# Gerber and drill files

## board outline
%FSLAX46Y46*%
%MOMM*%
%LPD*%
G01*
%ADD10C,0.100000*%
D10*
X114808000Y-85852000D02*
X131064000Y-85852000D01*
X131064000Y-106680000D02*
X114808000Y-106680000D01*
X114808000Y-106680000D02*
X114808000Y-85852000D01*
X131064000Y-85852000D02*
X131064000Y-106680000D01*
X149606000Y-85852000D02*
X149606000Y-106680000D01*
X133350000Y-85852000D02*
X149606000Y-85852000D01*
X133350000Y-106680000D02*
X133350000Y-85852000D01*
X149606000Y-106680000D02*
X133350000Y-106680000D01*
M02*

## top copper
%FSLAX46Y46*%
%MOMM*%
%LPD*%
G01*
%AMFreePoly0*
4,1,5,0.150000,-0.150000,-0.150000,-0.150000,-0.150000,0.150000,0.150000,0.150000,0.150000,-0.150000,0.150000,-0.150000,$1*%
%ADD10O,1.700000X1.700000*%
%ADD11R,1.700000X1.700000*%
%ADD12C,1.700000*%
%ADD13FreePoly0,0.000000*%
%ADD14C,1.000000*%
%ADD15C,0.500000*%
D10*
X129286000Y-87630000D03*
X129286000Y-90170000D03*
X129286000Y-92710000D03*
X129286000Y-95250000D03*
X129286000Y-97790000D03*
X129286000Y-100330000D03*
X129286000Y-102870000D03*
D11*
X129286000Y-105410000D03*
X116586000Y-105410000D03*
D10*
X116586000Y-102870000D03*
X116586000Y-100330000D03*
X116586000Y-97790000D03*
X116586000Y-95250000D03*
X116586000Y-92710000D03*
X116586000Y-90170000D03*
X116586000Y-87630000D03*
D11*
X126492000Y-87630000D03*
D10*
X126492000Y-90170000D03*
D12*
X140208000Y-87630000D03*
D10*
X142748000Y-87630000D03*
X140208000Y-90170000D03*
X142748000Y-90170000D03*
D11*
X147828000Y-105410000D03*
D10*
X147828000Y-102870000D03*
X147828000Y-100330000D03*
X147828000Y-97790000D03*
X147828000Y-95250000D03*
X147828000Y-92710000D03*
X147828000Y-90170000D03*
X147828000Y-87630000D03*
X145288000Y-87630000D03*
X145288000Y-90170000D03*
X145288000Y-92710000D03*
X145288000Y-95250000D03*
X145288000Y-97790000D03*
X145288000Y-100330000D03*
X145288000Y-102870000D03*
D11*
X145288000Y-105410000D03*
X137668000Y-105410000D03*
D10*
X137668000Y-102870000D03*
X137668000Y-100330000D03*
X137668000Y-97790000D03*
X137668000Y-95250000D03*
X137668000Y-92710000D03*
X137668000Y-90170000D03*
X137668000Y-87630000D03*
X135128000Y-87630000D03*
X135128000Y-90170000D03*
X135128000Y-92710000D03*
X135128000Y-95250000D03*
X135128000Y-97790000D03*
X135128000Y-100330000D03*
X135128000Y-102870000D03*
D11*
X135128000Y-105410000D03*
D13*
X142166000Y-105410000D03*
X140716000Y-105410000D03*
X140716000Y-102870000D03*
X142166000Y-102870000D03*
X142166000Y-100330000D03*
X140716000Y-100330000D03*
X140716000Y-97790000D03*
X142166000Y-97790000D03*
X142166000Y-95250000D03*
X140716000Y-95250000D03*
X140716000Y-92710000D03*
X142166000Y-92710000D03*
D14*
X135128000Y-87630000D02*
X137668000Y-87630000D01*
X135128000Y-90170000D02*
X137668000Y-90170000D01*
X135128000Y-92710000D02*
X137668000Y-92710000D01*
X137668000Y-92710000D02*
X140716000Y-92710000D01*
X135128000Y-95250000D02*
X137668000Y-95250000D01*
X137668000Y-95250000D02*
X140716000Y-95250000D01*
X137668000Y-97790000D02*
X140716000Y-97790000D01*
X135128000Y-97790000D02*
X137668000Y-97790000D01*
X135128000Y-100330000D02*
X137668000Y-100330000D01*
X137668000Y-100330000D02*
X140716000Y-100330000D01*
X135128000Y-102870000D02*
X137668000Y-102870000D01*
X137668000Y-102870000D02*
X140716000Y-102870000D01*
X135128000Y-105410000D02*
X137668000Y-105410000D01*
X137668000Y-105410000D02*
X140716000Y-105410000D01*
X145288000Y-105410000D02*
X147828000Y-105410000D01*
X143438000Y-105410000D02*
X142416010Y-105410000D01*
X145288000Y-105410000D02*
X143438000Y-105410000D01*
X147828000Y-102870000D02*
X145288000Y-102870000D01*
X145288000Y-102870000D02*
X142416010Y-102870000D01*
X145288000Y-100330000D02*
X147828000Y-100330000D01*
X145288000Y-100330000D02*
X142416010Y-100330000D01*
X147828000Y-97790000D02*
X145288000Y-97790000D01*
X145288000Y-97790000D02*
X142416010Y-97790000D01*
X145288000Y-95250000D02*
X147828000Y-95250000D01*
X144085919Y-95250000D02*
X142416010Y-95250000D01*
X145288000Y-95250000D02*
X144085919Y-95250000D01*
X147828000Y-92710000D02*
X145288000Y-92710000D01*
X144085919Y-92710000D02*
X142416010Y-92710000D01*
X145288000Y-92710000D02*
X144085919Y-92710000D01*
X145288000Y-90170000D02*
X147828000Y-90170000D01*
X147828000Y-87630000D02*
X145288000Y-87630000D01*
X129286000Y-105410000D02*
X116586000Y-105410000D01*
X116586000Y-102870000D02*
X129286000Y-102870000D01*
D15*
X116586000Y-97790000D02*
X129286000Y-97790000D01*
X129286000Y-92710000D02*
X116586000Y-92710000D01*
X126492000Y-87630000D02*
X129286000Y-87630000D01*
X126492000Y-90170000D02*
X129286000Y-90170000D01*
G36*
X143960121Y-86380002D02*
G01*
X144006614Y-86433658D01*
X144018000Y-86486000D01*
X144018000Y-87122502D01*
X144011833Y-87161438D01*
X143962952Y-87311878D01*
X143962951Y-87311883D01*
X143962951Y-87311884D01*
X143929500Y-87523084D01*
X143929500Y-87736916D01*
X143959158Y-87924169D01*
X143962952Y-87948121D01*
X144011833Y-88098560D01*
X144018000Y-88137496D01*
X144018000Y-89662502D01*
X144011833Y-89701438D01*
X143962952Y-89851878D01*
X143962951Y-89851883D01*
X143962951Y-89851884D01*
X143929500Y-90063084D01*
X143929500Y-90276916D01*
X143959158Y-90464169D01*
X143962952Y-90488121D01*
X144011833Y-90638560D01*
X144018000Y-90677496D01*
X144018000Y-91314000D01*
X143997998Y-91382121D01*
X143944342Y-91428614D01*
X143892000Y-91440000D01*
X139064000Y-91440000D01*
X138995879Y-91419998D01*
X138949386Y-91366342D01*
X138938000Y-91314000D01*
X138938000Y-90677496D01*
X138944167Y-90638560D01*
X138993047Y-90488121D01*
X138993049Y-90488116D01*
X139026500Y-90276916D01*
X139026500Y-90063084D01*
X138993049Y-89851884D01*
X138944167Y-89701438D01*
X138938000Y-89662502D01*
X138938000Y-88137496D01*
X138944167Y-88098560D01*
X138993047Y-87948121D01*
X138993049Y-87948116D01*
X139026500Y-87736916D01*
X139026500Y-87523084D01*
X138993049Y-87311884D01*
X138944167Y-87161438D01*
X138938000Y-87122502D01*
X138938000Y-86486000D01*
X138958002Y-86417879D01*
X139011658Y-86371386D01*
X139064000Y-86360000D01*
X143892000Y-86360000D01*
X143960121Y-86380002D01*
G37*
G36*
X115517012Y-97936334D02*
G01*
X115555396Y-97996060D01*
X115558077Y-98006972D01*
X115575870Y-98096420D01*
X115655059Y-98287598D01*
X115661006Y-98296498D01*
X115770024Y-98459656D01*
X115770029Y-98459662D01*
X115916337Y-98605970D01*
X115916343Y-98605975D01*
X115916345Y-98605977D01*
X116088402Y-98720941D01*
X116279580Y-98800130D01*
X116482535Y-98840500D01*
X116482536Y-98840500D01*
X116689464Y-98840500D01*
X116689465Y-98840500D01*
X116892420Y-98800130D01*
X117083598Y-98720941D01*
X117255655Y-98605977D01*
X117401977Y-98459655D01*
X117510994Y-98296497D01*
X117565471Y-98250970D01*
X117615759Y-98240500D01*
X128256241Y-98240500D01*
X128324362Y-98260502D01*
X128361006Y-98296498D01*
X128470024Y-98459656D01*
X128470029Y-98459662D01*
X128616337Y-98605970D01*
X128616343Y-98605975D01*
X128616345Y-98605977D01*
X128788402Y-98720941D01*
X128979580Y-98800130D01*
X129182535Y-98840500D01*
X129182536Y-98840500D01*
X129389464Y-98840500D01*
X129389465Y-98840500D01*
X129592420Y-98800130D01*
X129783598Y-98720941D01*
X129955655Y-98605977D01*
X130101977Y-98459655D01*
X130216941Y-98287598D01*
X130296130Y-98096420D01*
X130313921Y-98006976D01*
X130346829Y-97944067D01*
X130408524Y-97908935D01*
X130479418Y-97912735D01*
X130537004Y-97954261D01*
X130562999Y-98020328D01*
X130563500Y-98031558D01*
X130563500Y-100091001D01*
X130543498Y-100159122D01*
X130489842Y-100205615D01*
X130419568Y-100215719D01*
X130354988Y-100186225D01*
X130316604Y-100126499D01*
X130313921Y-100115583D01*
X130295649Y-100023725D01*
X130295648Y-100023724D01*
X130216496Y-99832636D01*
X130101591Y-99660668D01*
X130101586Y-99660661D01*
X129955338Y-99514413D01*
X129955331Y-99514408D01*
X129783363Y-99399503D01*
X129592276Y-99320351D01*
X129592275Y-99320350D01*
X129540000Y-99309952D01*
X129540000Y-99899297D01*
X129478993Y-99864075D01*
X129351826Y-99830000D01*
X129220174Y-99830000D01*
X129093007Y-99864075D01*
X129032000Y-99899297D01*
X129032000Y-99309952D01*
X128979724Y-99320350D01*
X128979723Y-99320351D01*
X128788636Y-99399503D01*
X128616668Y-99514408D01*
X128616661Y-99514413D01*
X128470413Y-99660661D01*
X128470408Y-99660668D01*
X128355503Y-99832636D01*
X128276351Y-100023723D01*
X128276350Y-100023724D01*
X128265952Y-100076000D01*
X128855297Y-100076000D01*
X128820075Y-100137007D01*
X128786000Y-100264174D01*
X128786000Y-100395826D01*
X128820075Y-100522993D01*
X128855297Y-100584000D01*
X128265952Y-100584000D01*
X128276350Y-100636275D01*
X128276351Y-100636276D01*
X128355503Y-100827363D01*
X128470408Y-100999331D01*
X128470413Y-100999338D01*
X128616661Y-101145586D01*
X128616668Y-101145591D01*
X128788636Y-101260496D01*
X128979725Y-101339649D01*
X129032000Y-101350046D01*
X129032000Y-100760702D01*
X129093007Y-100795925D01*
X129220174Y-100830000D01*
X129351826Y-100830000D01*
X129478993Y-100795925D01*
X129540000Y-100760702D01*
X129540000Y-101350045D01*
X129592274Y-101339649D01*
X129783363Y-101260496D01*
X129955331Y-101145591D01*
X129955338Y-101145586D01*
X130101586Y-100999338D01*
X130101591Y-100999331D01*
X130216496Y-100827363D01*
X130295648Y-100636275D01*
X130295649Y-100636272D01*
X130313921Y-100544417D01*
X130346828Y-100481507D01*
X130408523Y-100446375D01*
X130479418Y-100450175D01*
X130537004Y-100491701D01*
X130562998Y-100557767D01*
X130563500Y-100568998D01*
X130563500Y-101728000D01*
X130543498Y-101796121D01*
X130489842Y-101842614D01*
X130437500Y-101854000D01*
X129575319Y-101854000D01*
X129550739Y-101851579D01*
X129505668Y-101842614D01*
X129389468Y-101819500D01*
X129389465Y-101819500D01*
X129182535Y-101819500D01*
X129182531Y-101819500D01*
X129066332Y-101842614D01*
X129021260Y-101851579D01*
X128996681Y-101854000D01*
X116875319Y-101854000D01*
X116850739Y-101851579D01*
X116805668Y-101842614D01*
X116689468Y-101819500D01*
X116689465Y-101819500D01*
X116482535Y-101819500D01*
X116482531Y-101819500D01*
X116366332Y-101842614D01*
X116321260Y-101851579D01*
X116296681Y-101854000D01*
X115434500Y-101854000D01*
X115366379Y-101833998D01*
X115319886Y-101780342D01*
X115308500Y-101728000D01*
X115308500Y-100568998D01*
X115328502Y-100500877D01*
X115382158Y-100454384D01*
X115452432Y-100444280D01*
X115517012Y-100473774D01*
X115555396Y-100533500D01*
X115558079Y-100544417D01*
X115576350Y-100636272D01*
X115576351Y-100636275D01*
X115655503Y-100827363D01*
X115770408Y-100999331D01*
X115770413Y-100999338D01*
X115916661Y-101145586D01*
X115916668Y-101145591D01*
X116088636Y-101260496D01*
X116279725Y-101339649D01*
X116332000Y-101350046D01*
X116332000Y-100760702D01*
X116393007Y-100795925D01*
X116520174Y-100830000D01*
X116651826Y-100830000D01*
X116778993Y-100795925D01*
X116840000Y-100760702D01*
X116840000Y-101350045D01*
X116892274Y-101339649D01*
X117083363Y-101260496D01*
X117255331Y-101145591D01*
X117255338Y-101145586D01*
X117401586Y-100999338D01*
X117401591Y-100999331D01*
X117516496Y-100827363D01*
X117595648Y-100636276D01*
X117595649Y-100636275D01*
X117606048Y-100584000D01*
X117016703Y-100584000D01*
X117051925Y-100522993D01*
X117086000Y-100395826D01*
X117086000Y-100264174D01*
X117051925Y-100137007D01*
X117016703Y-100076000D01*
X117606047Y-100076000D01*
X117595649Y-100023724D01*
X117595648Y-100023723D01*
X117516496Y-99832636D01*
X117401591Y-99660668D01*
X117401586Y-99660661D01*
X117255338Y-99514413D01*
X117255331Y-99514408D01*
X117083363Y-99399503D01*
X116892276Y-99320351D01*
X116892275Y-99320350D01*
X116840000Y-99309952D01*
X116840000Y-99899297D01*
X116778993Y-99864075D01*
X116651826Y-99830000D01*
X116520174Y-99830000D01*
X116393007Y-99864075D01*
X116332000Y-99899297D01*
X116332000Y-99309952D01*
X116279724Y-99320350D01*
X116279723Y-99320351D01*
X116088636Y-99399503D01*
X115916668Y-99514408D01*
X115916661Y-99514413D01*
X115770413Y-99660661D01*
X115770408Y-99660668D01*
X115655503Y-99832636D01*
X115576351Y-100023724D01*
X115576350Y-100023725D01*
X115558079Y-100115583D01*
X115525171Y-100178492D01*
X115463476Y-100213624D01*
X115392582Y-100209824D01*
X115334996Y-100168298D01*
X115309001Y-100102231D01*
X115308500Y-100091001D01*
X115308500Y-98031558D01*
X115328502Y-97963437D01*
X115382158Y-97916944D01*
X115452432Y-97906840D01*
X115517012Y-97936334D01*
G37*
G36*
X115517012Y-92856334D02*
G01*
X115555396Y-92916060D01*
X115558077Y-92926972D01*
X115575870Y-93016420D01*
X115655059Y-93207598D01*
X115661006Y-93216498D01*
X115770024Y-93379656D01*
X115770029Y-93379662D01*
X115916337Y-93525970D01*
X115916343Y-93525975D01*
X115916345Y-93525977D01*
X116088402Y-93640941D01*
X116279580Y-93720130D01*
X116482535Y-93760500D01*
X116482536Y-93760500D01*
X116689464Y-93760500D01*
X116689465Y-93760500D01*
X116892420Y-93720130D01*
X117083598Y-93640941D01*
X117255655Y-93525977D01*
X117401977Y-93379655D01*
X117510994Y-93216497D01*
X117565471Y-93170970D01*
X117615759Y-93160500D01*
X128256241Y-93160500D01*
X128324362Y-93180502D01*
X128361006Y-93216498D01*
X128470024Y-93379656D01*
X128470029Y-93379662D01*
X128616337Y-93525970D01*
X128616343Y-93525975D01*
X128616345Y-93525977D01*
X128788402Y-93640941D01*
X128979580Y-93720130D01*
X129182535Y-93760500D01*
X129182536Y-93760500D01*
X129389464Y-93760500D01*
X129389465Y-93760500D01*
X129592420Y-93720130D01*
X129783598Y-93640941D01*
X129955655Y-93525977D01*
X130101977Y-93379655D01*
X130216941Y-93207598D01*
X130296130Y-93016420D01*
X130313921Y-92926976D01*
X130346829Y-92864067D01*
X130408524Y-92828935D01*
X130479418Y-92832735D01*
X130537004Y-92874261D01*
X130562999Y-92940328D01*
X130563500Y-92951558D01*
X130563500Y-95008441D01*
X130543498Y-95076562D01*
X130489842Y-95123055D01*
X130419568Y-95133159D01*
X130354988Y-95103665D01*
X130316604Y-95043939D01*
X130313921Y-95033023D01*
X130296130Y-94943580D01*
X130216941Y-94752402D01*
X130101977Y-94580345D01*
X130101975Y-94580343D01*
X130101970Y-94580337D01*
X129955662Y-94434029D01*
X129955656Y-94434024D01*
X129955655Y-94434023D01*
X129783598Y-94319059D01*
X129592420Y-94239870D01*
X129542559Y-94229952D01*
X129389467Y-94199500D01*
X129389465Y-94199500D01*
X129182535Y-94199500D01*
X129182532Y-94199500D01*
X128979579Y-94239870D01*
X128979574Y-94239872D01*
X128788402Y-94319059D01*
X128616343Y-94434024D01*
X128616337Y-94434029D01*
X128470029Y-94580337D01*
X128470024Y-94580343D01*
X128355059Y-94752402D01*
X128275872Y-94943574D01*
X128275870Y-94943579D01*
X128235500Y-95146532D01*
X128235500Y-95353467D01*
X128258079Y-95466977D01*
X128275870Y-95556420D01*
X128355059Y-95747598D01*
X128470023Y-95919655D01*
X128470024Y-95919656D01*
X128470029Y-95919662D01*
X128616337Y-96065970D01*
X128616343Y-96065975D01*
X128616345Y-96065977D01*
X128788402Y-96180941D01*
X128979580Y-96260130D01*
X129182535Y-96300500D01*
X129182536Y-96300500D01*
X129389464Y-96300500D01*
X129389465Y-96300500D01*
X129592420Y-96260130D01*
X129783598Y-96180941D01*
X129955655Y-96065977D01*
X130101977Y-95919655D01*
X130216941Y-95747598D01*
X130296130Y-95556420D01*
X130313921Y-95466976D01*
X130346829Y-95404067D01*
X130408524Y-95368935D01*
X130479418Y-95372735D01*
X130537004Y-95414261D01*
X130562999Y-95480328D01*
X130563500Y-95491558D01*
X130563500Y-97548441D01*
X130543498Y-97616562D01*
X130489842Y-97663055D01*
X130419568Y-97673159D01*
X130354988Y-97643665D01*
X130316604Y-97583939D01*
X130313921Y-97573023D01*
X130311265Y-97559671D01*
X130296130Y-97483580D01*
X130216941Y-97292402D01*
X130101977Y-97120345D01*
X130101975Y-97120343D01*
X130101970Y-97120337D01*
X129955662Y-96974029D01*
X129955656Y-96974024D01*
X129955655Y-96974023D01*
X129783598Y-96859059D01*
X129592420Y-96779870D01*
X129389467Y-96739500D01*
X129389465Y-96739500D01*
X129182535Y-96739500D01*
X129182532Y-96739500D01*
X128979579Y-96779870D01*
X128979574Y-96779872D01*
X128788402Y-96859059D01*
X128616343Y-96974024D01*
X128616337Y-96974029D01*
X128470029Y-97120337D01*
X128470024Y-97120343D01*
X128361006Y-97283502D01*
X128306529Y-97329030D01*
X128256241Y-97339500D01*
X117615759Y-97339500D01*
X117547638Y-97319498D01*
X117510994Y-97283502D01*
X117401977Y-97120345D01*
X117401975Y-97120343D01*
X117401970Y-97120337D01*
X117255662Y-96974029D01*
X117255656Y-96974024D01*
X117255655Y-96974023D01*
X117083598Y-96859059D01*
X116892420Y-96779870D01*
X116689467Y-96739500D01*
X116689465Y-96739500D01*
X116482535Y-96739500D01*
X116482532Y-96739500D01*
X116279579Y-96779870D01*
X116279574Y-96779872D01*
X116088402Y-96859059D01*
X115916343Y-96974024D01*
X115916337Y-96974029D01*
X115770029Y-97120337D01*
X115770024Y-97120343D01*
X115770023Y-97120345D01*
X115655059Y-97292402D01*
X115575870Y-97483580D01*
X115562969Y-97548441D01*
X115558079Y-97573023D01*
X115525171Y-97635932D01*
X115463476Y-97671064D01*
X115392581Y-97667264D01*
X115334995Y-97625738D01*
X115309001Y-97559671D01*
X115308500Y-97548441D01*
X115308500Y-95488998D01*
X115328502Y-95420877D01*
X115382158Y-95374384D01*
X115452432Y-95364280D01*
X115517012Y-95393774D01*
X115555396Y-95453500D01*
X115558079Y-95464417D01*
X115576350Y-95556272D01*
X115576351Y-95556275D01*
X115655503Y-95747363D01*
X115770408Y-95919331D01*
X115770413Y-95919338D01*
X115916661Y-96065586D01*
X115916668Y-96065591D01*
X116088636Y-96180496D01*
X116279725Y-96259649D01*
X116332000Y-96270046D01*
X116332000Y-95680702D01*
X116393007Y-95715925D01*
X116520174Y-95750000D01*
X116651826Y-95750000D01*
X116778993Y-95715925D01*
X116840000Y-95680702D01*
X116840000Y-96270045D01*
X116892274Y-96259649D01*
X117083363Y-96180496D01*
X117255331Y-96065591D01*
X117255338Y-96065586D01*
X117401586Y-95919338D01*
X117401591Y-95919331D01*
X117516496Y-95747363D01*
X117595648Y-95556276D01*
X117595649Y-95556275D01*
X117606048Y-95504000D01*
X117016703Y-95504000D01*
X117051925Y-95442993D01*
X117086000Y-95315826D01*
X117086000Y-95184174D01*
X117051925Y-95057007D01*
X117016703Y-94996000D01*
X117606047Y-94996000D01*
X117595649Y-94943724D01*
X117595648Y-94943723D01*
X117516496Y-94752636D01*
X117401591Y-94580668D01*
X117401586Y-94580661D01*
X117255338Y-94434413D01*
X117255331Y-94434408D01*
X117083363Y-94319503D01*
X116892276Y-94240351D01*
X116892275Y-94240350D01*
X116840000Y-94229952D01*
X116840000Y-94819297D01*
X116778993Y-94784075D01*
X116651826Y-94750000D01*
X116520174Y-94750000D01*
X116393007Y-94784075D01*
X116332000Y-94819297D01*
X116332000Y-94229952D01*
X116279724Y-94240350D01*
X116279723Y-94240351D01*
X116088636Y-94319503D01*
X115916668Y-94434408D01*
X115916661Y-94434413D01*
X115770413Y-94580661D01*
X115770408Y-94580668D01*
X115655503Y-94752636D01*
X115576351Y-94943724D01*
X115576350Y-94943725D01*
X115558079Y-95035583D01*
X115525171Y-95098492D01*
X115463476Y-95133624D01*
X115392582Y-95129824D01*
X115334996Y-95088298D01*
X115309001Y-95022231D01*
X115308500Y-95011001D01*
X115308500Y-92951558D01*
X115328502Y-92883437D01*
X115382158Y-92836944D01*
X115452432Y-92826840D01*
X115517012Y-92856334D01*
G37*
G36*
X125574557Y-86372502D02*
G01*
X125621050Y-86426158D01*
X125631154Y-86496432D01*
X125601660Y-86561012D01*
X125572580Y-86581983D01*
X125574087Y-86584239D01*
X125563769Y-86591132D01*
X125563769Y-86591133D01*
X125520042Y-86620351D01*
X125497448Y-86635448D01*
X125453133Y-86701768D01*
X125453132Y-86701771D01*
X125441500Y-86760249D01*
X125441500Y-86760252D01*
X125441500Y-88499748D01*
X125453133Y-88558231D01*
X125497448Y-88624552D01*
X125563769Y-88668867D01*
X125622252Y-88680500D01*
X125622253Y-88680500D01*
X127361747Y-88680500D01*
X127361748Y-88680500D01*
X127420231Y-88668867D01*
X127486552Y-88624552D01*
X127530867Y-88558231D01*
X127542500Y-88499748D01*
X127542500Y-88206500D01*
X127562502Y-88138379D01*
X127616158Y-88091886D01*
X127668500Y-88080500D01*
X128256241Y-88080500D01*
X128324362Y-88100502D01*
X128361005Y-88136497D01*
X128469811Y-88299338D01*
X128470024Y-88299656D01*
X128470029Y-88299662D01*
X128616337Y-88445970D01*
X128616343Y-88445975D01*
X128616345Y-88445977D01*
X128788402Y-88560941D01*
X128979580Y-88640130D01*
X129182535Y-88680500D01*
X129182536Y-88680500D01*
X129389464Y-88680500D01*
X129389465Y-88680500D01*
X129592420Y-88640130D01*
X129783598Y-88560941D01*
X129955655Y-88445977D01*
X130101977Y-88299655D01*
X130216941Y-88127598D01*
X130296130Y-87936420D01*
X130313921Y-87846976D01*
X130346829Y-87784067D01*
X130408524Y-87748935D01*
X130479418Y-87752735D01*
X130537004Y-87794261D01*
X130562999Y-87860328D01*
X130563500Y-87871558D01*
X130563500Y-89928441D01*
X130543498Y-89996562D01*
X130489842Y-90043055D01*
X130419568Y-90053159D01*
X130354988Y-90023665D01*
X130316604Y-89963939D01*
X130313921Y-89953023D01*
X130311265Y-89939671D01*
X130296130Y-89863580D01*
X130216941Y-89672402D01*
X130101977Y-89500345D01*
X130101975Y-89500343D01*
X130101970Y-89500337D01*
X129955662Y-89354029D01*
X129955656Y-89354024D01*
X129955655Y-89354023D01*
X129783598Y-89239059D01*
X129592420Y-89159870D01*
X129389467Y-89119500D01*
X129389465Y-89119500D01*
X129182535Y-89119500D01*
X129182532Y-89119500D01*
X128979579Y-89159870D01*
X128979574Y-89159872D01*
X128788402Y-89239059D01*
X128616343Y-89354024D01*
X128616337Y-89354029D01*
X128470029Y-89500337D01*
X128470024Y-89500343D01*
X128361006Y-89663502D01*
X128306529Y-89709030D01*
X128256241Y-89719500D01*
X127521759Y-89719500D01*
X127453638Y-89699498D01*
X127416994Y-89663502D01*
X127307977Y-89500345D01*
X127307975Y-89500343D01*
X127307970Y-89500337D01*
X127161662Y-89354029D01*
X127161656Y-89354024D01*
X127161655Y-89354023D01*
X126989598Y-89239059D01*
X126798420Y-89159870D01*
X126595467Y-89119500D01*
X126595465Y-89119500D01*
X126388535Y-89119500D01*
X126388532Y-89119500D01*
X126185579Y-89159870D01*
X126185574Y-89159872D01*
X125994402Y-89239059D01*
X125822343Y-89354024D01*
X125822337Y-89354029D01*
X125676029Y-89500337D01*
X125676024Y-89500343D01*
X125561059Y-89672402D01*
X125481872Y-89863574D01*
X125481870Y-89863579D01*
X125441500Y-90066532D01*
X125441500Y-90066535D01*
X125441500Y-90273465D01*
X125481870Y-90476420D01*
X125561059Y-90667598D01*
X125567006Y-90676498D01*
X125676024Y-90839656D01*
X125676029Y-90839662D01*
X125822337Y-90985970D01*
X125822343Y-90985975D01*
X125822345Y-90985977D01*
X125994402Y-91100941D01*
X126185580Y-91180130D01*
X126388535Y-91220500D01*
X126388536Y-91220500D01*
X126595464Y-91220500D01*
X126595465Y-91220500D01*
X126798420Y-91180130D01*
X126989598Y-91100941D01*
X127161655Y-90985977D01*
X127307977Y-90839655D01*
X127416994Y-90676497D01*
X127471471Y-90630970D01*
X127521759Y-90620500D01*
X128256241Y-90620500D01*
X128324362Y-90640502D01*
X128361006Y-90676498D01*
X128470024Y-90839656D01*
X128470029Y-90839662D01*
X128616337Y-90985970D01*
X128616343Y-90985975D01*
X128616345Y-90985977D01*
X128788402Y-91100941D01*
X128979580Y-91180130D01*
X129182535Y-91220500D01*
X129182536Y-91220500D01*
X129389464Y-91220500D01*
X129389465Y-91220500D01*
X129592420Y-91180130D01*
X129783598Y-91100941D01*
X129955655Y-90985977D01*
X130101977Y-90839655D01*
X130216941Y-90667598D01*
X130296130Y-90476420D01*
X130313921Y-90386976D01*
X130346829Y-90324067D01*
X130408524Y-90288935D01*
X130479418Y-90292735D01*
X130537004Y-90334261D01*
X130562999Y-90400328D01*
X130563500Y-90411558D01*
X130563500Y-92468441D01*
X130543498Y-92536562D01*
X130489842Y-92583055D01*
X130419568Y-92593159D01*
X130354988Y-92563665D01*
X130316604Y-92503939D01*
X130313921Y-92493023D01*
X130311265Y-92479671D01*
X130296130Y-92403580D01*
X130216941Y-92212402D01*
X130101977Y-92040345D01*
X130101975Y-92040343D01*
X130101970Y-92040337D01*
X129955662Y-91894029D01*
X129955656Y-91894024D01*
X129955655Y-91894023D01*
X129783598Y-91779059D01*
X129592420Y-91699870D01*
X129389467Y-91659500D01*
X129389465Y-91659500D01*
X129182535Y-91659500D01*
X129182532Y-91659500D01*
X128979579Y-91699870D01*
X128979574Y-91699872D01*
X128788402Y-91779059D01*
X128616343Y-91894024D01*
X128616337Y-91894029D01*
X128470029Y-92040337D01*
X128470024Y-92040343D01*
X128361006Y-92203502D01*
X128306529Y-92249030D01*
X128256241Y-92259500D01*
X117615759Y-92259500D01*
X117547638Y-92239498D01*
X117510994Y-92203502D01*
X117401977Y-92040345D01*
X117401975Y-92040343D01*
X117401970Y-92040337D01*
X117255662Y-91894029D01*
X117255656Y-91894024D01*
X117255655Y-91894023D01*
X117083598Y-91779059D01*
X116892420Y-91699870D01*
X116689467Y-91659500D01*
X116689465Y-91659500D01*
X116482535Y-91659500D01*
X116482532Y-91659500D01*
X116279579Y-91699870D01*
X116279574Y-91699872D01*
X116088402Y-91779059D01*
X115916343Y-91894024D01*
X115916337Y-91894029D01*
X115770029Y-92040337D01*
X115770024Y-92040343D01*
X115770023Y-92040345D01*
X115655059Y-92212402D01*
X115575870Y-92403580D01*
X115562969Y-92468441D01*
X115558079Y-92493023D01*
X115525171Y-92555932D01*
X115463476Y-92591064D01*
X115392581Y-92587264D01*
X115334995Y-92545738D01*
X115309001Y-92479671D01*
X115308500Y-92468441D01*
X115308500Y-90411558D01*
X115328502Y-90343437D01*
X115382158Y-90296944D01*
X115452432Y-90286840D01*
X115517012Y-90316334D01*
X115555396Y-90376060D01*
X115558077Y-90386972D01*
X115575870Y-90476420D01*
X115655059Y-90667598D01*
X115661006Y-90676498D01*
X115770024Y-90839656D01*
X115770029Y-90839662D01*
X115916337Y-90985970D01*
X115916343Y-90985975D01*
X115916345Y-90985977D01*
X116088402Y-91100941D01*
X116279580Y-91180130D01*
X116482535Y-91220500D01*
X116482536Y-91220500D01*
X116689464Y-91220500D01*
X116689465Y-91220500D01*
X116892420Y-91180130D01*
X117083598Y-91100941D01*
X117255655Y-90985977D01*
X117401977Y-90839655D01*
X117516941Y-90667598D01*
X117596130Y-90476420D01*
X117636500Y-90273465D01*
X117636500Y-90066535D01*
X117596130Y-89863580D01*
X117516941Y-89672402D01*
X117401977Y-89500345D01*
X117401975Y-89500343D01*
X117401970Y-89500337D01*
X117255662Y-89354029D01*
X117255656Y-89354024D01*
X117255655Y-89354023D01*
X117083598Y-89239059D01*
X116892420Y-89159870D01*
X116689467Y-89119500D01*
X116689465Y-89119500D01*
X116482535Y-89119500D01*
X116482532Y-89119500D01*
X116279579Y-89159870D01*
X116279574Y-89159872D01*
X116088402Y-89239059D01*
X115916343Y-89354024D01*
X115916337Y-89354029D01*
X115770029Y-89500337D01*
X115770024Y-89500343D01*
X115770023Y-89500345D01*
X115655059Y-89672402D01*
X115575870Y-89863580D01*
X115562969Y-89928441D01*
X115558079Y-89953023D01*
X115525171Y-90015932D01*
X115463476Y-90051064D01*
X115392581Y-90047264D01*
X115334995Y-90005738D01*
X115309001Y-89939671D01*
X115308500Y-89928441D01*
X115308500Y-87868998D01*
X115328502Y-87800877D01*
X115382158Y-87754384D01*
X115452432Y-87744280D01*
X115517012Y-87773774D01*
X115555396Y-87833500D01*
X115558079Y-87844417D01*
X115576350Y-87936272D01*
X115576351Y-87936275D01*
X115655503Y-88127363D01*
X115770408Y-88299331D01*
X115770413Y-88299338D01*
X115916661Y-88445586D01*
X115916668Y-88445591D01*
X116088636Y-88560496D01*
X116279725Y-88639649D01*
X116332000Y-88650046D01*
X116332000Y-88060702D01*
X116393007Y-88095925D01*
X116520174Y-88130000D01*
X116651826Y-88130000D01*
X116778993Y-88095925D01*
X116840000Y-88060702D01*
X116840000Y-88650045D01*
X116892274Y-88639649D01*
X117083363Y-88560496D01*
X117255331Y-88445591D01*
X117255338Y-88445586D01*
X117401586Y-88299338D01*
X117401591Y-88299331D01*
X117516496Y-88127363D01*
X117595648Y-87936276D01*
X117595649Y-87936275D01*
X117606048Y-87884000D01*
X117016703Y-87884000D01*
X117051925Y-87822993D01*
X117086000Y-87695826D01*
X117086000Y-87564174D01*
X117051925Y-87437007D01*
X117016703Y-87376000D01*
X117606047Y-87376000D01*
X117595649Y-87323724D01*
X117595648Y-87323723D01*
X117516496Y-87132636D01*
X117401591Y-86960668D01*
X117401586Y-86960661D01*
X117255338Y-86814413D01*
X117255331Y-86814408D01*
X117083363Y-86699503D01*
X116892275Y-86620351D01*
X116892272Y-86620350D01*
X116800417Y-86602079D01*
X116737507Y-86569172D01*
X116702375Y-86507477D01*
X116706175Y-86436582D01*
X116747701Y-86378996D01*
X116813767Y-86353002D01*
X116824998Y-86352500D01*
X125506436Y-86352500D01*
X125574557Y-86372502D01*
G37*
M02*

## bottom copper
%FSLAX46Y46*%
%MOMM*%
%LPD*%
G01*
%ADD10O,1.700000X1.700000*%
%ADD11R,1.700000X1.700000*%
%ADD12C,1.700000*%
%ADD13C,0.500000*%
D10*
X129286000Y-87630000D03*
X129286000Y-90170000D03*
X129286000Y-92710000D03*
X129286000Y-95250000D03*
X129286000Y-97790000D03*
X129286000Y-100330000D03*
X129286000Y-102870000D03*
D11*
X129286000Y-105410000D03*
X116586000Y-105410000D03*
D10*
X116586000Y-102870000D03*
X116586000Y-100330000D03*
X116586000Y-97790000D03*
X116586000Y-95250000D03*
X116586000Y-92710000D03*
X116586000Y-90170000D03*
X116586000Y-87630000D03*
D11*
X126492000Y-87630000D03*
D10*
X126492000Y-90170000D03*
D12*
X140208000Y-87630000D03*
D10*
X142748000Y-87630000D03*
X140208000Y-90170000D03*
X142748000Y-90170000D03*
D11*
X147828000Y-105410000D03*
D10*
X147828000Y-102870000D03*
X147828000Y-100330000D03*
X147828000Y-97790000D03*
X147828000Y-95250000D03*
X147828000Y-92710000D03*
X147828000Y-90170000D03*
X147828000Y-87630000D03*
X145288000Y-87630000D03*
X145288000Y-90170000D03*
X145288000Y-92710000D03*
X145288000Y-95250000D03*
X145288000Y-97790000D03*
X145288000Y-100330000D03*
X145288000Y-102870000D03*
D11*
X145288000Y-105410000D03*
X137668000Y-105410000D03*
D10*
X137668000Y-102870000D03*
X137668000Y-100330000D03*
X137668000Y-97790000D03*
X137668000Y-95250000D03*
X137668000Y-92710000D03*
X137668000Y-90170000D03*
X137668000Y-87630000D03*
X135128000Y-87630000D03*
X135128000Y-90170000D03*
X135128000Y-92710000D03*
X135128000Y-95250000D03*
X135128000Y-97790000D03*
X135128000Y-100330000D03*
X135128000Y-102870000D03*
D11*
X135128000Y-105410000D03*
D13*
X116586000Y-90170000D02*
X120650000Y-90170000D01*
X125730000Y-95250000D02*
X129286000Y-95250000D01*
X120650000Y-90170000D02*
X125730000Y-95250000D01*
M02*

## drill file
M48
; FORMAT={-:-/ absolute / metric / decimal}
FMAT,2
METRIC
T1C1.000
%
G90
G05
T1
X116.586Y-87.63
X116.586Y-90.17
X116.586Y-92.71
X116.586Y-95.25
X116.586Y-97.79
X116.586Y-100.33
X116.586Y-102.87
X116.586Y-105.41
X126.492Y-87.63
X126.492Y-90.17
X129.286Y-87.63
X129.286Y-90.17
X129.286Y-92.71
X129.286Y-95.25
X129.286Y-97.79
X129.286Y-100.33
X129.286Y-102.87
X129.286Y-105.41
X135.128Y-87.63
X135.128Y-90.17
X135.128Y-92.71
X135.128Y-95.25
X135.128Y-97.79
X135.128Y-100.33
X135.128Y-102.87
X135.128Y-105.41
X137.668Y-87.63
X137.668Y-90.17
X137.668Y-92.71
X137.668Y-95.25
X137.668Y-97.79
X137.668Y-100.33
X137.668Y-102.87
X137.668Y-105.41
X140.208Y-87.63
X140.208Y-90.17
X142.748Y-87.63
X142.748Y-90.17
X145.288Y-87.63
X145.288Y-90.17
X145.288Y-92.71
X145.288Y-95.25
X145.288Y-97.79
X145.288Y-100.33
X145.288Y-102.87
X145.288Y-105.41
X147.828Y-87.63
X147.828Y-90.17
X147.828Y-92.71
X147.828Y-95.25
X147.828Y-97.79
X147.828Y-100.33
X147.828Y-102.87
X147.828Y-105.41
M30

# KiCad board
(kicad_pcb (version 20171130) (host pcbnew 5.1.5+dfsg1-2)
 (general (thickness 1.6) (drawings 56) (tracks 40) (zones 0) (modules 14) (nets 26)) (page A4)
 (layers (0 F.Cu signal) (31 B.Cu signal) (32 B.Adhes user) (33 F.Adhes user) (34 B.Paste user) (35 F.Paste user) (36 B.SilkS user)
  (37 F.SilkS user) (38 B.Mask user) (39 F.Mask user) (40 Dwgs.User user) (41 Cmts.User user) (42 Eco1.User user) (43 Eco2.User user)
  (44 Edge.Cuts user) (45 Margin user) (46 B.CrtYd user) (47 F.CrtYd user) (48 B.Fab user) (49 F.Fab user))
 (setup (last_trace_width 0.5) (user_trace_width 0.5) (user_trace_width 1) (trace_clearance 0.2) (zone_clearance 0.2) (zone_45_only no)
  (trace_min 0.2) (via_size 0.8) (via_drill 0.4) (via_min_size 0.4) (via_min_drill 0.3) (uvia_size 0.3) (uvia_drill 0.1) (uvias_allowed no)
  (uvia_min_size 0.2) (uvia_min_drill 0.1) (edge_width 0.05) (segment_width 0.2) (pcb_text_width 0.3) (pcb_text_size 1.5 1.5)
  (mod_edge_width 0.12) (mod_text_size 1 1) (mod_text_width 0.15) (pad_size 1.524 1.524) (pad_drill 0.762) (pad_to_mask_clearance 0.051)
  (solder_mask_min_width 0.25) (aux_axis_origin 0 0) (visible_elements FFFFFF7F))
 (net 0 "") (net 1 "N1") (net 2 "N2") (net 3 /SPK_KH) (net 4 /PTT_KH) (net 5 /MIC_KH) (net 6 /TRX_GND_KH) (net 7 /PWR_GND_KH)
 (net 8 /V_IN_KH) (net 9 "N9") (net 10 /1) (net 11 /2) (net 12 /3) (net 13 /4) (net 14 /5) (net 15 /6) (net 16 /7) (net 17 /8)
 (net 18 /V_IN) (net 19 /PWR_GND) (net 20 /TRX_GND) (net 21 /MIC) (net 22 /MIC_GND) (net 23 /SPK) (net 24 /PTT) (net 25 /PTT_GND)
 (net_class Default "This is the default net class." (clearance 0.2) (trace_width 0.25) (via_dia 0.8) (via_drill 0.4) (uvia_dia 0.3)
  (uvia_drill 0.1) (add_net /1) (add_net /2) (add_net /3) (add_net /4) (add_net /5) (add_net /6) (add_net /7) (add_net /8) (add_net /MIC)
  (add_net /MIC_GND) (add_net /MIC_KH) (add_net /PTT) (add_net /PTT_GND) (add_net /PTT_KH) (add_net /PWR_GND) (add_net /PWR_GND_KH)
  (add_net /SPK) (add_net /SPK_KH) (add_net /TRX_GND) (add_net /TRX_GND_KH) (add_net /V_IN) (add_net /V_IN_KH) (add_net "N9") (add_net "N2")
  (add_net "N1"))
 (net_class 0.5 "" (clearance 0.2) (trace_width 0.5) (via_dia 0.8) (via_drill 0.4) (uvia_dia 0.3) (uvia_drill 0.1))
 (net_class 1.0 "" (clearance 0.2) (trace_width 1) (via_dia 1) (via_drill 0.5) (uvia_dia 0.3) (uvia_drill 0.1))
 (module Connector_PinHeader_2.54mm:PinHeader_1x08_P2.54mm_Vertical (layer F.Cu) (at 129.286 105.41 180)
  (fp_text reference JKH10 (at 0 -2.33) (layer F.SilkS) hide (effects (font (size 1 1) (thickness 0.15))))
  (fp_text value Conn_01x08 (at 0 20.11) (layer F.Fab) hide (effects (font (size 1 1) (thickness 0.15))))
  (pad 8 thru_hole oval (at 0 17.78 180) (size 1.7 1.7) (drill 1) (layers *.Cu *.Mask) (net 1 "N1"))
  (pad 7 thru_hole oval (at 0 15.24 180) (size 1.7 1.7) (drill 1) (layers *.Cu *.Mask) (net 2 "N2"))
  (pad 6 thru_hole oval (at 0 12.7 180) (size 1.7 1.7) (drill 1) (layers *.Cu *.Mask) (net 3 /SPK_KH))
  (pad 5 thru_hole oval (at 0 10.16 180) (size 1.7 1.7) (drill 1) (layers *.Cu *.Mask) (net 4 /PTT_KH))
  (pad 4 thru_hole oval (at 0 7.62 180) (size 1.7 1.7) (drill 1) (layers *.Cu *.Mask) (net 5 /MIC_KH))
  (pad 3 thru_hole oval (at 0 5.08 180) (size 1.7 1.7) (drill 1) (layers *.Cu *.Mask) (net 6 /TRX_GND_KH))
  (pad 2 thru_hole oval (at 0 2.54 180) (size 1.7 1.7) (drill 1) (layers *.Cu *.Mask) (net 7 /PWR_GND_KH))
  (pad 1 thru_hole rect (at 0 0 180) (size 1.7 1.7) (drill 1) (layers *.Cu *.Mask) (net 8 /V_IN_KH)))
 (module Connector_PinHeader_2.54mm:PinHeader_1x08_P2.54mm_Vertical (layer F.Cu) (at 116.586 105.41 180)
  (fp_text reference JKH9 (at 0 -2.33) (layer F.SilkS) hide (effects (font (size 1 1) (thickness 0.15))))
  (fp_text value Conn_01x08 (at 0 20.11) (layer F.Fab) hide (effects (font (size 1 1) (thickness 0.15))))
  (pad 1 thru_hole rect (at 0 0 180) (size 1.7 1.7) (drill 1) (layers *.Cu *.Mask) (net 8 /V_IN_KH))
  (pad 2 thru_hole oval (at 0 2.54 180) (size 1.7 1.7) (drill 1) (layers *.Cu *.Mask) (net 7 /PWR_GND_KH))
  (pad 3 thru_hole oval (at 0 5.08 180) (size 1.7 1.7) (drill 1) (layers *.Cu *.Mask) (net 6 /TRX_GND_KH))
  (pad 4 thru_hole oval (at 0 7.62 180) (size 1.7 1.7) (drill 1) (layers *.Cu *.Mask) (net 5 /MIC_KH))
  (pad 5 thru_hole oval (at 0 10.16 180) (size 1.7 1.7) (drill 1) (layers *.Cu *.Mask) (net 6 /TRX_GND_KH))
  (pad 6 thru_hole oval (at 0 12.7 180) (size 1.7 1.7) (drill 1) (layers *.Cu *.Mask) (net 3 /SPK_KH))
  (pad 7 thru_hole oval (at 0 15.24 180) (size 1.7 1.7) (drill 1) (layers *.Cu *.Mask) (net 4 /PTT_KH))
  (pad 8 thru_hole oval (at 0 17.78 180) (size 1.7 1.7) (drill 1) (layers *.Cu *.Mask) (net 6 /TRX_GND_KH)))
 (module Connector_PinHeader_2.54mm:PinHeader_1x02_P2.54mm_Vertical (layer F.Cu) (at 126.492 87.63)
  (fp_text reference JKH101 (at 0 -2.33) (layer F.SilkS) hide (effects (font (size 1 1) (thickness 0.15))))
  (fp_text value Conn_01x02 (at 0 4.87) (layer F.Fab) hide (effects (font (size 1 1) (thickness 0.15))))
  (pad 1 thru_hole rect (at 0 0) (size 1.7 1.7) (drill 1) (layers *.Cu *.Mask) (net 1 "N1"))
  (pad 2 thru_hole oval (at 0 2.54) (size 1.7 1.7) (drill 1) (layers *.Cu *.Mask) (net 2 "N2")))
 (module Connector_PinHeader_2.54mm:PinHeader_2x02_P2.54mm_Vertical (layer F.Cu) (at 140.208 87.63)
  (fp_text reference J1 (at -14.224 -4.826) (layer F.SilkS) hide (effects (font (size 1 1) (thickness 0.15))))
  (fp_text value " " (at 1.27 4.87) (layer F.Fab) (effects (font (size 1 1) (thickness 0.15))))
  (pad 1 thru_hole circle (at 0 0) (size 1.7 1.7) (drill 1) (layers *.Cu *.Mask) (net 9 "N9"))
  (pad 2 thru_hole oval (at 2.54 0) (size 1.7 1.7) (drill 1) (layers *.Cu *.Mask) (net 9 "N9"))
  (pad 3 thru_hole oval (at 0 2.54) (size 1.7 1.7) (drill 1) (layers *.Cu *.Mask) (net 9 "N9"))
  (pad 4 thru_hole oval (at 2.54 2.54) (size 1.7 1.7) (drill 1) (layers *.Cu *.Mask) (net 9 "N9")))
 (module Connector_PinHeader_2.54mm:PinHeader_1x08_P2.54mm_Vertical (layer F.Cu) (at 147.828 105.41 180)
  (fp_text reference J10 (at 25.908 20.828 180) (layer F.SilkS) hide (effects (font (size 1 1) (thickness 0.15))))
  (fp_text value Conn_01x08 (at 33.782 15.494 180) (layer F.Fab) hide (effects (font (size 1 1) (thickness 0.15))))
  (pad 1 thru_hole rect (at 0 0 180) (size 1.7 1.7) (drill 1) (layers *.Cu *.Mask) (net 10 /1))
  (pad 2 thru_hole oval (at 0 2.54 180) (size 1.7 1.7) (drill 1) (layers *.Cu *.Mask) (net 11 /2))
  (pad 3 thru_hole oval (at 0 5.08 180) (size 1.7 1.7) (drill 1) (layers *.Cu *.Mask) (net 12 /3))
  (pad 4 thru_hole oval (at 0 7.62 180) (size 1.7 1.7) (drill 1) (layers *.Cu *.Mask) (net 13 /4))
  (pad 5 thru_hole oval (at 0 10.16 180) (size 1.7 1.7) (drill 1) (layers *.Cu *.Mask) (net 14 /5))
  (pad 6 thru_hole oval (at 0 12.7 180) (size 1.7 1.7) (drill 1) (layers *.Cu *.Mask) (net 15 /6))
  (pad 7 thru_hole oval (at 0 15.24 180) (size 1.7 1.7) (drill 1) (layers *.Cu *.Mask) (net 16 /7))
  (pad 8 thru_hole oval (at 0 17.78 180) (size 1.7 1.7) (drill 1) (layers *.Cu *.Mask) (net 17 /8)))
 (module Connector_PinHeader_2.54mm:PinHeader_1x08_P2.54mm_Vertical (layer F.Cu) (at 145.288 105.41 180)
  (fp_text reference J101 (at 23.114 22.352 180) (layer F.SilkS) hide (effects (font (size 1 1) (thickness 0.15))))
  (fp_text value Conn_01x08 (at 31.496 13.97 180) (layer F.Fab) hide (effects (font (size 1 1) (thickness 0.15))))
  (pad 8 thru_hole oval (at 0 17.78 180) (size 1.7 1.7) (drill 1) (layers *.Cu *.Mask) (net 17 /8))
  (pad 7 thru_hole oval (at 0 15.24 180) (size 1.7 1.7) (drill 1) (layers *.Cu *.Mask) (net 16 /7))
  (pad 6 thru_hole oval (at 0 12.7 180) (size 1.7 1.7) (drill 1) (layers *.Cu *.Mask) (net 15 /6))
  (pad 5 thru_hole oval (at 0 10.16 180) (size 1.7 1.7) (drill 1) (layers *.Cu *.Mask) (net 14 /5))
  (pad 4 thru_hole oval (at 0 7.62 180) (size 1.7 1.7) (drill 1) (layers *.Cu *.Mask) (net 13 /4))
  (pad 3 thru_hole oval (at 0 5.08 180) (size 1.7 1.7) (drill 1) (layers *.Cu *.Mask) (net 12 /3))
  (pad 2 thru_hole oval (at 0 2.54 180) (size 1.7 1.7) (drill 1) (layers *.Cu *.Mask) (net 11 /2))
  (pad 1 thru_hole rect (at 0 0 180) (size 1.7 1.7) (drill 1) (layers *.Cu *.Mask) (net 10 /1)))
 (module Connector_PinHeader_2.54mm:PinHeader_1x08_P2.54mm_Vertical (layer F.Cu) (at 137.668 105.41 180)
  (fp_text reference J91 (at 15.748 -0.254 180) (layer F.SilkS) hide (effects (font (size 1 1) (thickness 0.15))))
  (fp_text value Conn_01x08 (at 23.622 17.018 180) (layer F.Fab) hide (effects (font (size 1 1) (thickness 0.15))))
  (pad 1 thru_hole rect (at 0 0 180) (size 1.7 1.7) (drill 1) (layers *.Cu *.Mask) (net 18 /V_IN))
  (pad 2 thru_hole oval (at 0 2.54 180) (size 1.7 1.7) (drill 1) (layers *.Cu *.Mask) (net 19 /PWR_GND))
  (pad 3 thru_hole oval (at 0 5.08 180) (size 1.7 1.7) (drill 1) (layers *.Cu *.Mask) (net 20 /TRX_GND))
  (pad 4 thru_hole oval (at 0 7.62 180) (size 1.7 1.7) (drill 1) (layers *.Cu *.Mask) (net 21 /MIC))
  (pad 5 thru_hole oval (at 0 10.16 180) (size 1.7 1.7) (drill 1) (layers *.Cu *.Mask) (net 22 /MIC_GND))
  (pad 6 thru_hole oval (at 0 12.7 180) (size 1.7 1.7) (drill 1) (layers *.Cu *.Mask) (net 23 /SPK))
  (pad 7 thru_hole oval (at 0 15.24 180) (size 1.7 1.7) (drill 1) (layers *.Cu *.Mask) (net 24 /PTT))
  (pad 8 thru_hole oval (at 0 17.78 180) (size 1.7 1.7) (drill 1) (layers *.Cu *.Mask) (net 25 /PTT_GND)))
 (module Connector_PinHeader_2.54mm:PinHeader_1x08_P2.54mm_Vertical (layer F.Cu) (at 135.128 105.41 180)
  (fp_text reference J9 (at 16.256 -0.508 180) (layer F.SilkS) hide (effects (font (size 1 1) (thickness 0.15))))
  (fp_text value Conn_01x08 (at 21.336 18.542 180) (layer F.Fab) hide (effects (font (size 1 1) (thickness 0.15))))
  (pad 8 thru_hole oval (at 0 17.78 180) (size 1.7 1.7) (drill 1) (layers *.Cu *.Mask) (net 25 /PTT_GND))
  (pad 7 thru_hole oval (at 0 15.24 180) (size 1.7 1.7) (drill 1) (layers *.Cu *.Mask) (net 24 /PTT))
  (pad 6 thru_hole oval (at 0 12.7 180) (size 1.7 1.7) (drill 1) (layers *.Cu *.Mask) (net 23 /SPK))
  (pad 5 thru_hole oval (at 0 10.16 180) (size 1.7 1.7) (drill 1) (layers *.Cu *.Mask) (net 22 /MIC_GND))
  (pad 4 thru_hole oval (at 0 7.62 180) (size 1.7 1.7) (drill 1) (layers *.Cu *.Mask) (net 21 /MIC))
  (pad 3 thru_hole oval (at 0 5.08 180) (size 1.7 1.7) (drill 1) (layers *.Cu *.Mask) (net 20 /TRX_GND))
  (pad 2 thru_hole oval (at 0 2.54 180) (size 1.7 1.7) (drill 1) (layers *.Cu *.Mask) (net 19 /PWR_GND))
  (pad 1 thru_hole rect (at 0 0 180) (size 1.7 1.7) (drill 1) (layers *.Cu *.Mask) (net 18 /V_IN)))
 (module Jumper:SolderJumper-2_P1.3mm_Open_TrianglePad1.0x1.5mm (layer F.Cu) (at 141.441 105.41)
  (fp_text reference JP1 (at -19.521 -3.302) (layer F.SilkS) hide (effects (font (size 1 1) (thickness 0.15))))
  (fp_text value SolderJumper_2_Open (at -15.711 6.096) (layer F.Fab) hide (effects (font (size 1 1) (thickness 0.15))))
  (pad 2 smd custom (at 0.725 0) (size 0.3 0.3) (layers F.Cu F.Mask) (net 10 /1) (zone_connect 2)
   (options (clearance outline) (anchor rect)) (primitives))
  (pad 1 smd custom (at -0.725 0) (size 0.3 0.3) (layers F.Cu F.Mask) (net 18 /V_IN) (zone_connect 2)
   (options (clearance outline) (anchor rect)) (primitives)))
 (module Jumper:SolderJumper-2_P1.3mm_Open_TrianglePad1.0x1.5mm (layer F.Cu) (at 141.441 102.87)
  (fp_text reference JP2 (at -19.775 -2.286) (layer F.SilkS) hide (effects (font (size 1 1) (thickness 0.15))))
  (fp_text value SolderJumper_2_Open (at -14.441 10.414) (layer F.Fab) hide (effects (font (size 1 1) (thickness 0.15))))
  (pad 1 smd custom (at -0.725 0) (size 0.3 0.3) (layers F.Cu F.Mask) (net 19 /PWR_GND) (zone_connect 2)
   (options (clearance outline) (anchor rect)) (primitives))
  (pad 2 smd custom (at 0.725 0) (size 0.3 0.3) (layers F.Cu F.Mask) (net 11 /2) (zone_connect 2)
   (options (clearance outline) (anchor rect)) (primitives)))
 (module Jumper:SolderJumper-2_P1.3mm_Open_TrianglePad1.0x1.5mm (layer F.Cu) (at 141.441 100.33)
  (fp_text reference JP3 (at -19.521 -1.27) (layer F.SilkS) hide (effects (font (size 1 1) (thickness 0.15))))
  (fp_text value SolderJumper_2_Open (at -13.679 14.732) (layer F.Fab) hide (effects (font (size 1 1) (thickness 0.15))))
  (pad 2 smd custom (at 0.725 0) (size 0.3 0.3) (layers F.Cu F.Mask) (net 12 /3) (zone_connect 2)
   (options (clearance outline) (anchor rect)) (primitives))
  (pad 1 smd custom (at -0.725 0) (size 0.3 0.3) (layers F.Cu F.Mask) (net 20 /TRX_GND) (zone_connect 2)
   (options (clearance outline) (anchor rect)) (primitives)))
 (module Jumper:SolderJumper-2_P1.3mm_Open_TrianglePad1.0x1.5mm (layer F.Cu) (at 141.441 97.79)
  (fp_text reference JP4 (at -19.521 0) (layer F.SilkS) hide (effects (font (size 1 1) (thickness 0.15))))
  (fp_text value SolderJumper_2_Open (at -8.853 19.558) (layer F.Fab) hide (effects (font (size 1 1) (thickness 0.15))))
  (pad 1 smd custom (at -0.725 0) (size 0.3 0.3) (layers F.Cu F.Mask) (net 21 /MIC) (zone_connect 2)
   (options (clearance outline) (anchor rect)) (primitives))
  (pad 2 smd custom (at 0.725 0) (size 0.3 0.3) (layers F.Cu F.Mask) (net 13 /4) (zone_connect 2)
   (options (clearance outline) (anchor rect)) (primitives)))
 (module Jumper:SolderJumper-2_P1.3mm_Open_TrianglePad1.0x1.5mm (layer F.Cu) (at 141.441 95.25)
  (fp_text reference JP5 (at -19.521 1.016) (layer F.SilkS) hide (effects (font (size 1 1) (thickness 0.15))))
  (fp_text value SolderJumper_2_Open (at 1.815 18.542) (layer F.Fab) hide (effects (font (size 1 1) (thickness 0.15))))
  (pad 2 smd custom (at 0.725 0) (size 0.3 0.3) (layers F.Cu F.Mask) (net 14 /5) (zone_connect 2)
   (options (clearance outline) (anchor rect)) (primitives))
  (pad 1 smd custom (at -0.725 0) (size 0.3 0.3) (layers F.Cu F.Mask) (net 22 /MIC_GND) (zone_connect 2)
   (options (clearance outline) (anchor rect)) (primitives)))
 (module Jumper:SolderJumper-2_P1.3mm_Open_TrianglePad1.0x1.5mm (layer F.Cu) (at 141.441 92.71)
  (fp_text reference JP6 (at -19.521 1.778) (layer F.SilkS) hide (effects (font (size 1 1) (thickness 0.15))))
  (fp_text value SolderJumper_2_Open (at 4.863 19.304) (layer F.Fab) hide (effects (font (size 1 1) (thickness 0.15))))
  (pad 1 smd custom (at -0.725 0) (size 0.3 0.3) (layers F.Cu F.Mask) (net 23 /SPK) (zone_connect 2)
   (options (clearance outline) (anchor rect)) (primitives))
  (pad 2 smd custom (at 0.725 0) (size 0.3 0.3) (layers F.Cu F.Mask) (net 15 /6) (zone_connect 2)
   (options (clearance outline) (anchor rect)) (primitives)))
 (gr_line (start 114.808 85.852) (end 131.064 85.852) (layer Edge.Cuts) (width 0.1))
 (gr_line (start 131.064 106.68) (end 114.808 106.68) (layer Edge.Cuts) (width 0.1))
 (gr_line (start 114.808 106.68) (end 114.808 85.852) (layer Edge.Cuts) (width 0.1))
 (gr_line (start 131.064 85.852) (end 131.064 106.68) (layer Edge.Cuts) (width 0.1))
 (gr_line (start 149.606 85.852) (end 149.606 106.68) (layer Edge.Cuts) (width 0.1))
 (gr_line (start 133.35 85.852) (end 149.606 85.852) (layer Edge.Cuts) (width 0.1))
 (gr_line (start 133.35 106.68) (end 133.35 85.852) (layer Edge.Cuts) (width 0.1))
 (gr_line (start 149.606 106.68) (end 133.35 106.68) (layer Edge.Cuts) (width 0.1))
 (segment (start 135.128 87.63) (end 137.668 87.63) (width 1) (layer F.Cu) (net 25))
 (segment (start 135.128 90.17) (end 137.668 90.17) (width 1) (layer F.Cu) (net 24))
 (segment (start 135.128 92.71) (end 137.668 92.71) (width 1) (layer F.Cu) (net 23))
 (segment (start 137.668 92.71) (end 140.716 92.71) (width 1) (layer F.Cu) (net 23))
 (segment (start 135.128 95.25) (end 137.668 95.25) (width 1) (layer F.Cu) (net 22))
 (segment (start 137.668 95.25) (end 140.716 95.25) (width 1) (layer F.Cu) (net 22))
 (segment (start 137.668 97.79) (end 140.716 97.79) (width 1) (layer F.Cu) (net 21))
 (segment (start 135.128 97.79) (end 137.668 97.79) (width 1) (layer F.Cu) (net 21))
 (segment (start 135.128 100.33) (end 137.668 100.33) (width 1) (layer F.Cu) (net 20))
 (segment (start 137.668 100.33) (end 140.716 100.33) (width 1) (layer F.Cu) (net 20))
 (segment (start 135.128 102.87) (end 137.668 102.87) (width 1) (layer F.Cu) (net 19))
 (segment (start 137.668 102.87) (end 140.716 102.87) (width 1) (layer F.Cu) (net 19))
 (segment (start 135.128 105.41) (end 137.668 105.41) (width 1) (layer F.Cu) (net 18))
 (segment (start 137.668 105.41) (end 140.716 105.41) (width 1) (layer F.Cu) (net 18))
 (segment (start 145.288 105.41) (end 147.828 105.41) (width 1) (layer F.Cu) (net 10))
 (segment (start 143.438 105.41) (end 142.41601 105.41) (width 1) (layer F.Cu) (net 10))
 (segment (start 145.288 105.41) (end 143.438 105.41) (width 1) (layer F.Cu) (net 10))
 (segment (start 147.828 102.87) (end 145.288 102.87) (width 1) (layer F.Cu) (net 11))
 (segment (start 145.288 102.87) (end 142.41601 102.87) (width 1) (layer F.Cu) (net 11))
 (segment (start 145.288 100.33) (end 147.828 100.33) (width 1) (layer F.Cu) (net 12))
 (segment (start 145.288 100.33) (end 142.41601 100.33) (width 1) (layer F.Cu) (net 12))
 (segment (start 147.828 97.79) (end 145.288 97.79) (width 1) (layer F.Cu) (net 13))
 (segment (start 145.288 97.79) (end 142.41601 97.79) (width 1) (layer F.Cu) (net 13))
 (segment (start 145.288 95.25) (end 147.828 95.25) (width 1) (layer F.Cu) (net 14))
 (segment (start 144.085919 95.25) (end 142.41601 95.25) (width 1) (layer F.Cu) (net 14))
 (segment (start 145.288 95.25) (end 144.085919 95.25) (width 1) (layer F.Cu) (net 14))
 (segment (start 147.828 92.71) (end 145.288 92.71) (width 1) (layer F.Cu) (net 15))
 (segment (start 144.085919 92.71) (end 142.41601 92.71) (width 1) (layer F.Cu) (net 15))
 (segment (start 145.288 92.71) (end 144.085919 92.71) (width 1) (layer F.Cu) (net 15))
 (segment (start 145.288 90.17) (end 147.828 90.17) (width 1) (layer F.Cu) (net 16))
 (segment (start 147.828 87.63) (end 145.288 87.63) (width 1) (layer F.Cu) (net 17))
 (segment (start 129.286 105.41) (end 116.586 105.41) (width 1) (layer F.Cu) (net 8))
 (segment (start 116.586 102.87) (end 129.286 102.87) (width 1) (layer F.Cu) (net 7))
 (segment (start 116.586 97.79) (end 129.286 97.79) (width 0.5) (layer F.Cu) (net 5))
 (segment (start 129.286 92.71) (end 116.586 92.71) (width 0.5) (layer F.Cu) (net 3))
 (segment (start 116.586 90.17) (end 120.65 90.17) (width 0.5) (layer B.Cu) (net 4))
 (segment (start 125.73 95.25) (end 129.286 95.25) (width 0.5) (layer B.Cu) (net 4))
 (segment (start 120.65 90.17) (end 125.73 95.25) (width 0.5) (layer B.Cu) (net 4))
 (segment (start 126.492 87.63) (end 129.286 87.63) (width 0.5) (layer F.Cu) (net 1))
 (segment (start 126.492 90.17) (end 129.286 90.17) (width 0.5) (layer F.Cu) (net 2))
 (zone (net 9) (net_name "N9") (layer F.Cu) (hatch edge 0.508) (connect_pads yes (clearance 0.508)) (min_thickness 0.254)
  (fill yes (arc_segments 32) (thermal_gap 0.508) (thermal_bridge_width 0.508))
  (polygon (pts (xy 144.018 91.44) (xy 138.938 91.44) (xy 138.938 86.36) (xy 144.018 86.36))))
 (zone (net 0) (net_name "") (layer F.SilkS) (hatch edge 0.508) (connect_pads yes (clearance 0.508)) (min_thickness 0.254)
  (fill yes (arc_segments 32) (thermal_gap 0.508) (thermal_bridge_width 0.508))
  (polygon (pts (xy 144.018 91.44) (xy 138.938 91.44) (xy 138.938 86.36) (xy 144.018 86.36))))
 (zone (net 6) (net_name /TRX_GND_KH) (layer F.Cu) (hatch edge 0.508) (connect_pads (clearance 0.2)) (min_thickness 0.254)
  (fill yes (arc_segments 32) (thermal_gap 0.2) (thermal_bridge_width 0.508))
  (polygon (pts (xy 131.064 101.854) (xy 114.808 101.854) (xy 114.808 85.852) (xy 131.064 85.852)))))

